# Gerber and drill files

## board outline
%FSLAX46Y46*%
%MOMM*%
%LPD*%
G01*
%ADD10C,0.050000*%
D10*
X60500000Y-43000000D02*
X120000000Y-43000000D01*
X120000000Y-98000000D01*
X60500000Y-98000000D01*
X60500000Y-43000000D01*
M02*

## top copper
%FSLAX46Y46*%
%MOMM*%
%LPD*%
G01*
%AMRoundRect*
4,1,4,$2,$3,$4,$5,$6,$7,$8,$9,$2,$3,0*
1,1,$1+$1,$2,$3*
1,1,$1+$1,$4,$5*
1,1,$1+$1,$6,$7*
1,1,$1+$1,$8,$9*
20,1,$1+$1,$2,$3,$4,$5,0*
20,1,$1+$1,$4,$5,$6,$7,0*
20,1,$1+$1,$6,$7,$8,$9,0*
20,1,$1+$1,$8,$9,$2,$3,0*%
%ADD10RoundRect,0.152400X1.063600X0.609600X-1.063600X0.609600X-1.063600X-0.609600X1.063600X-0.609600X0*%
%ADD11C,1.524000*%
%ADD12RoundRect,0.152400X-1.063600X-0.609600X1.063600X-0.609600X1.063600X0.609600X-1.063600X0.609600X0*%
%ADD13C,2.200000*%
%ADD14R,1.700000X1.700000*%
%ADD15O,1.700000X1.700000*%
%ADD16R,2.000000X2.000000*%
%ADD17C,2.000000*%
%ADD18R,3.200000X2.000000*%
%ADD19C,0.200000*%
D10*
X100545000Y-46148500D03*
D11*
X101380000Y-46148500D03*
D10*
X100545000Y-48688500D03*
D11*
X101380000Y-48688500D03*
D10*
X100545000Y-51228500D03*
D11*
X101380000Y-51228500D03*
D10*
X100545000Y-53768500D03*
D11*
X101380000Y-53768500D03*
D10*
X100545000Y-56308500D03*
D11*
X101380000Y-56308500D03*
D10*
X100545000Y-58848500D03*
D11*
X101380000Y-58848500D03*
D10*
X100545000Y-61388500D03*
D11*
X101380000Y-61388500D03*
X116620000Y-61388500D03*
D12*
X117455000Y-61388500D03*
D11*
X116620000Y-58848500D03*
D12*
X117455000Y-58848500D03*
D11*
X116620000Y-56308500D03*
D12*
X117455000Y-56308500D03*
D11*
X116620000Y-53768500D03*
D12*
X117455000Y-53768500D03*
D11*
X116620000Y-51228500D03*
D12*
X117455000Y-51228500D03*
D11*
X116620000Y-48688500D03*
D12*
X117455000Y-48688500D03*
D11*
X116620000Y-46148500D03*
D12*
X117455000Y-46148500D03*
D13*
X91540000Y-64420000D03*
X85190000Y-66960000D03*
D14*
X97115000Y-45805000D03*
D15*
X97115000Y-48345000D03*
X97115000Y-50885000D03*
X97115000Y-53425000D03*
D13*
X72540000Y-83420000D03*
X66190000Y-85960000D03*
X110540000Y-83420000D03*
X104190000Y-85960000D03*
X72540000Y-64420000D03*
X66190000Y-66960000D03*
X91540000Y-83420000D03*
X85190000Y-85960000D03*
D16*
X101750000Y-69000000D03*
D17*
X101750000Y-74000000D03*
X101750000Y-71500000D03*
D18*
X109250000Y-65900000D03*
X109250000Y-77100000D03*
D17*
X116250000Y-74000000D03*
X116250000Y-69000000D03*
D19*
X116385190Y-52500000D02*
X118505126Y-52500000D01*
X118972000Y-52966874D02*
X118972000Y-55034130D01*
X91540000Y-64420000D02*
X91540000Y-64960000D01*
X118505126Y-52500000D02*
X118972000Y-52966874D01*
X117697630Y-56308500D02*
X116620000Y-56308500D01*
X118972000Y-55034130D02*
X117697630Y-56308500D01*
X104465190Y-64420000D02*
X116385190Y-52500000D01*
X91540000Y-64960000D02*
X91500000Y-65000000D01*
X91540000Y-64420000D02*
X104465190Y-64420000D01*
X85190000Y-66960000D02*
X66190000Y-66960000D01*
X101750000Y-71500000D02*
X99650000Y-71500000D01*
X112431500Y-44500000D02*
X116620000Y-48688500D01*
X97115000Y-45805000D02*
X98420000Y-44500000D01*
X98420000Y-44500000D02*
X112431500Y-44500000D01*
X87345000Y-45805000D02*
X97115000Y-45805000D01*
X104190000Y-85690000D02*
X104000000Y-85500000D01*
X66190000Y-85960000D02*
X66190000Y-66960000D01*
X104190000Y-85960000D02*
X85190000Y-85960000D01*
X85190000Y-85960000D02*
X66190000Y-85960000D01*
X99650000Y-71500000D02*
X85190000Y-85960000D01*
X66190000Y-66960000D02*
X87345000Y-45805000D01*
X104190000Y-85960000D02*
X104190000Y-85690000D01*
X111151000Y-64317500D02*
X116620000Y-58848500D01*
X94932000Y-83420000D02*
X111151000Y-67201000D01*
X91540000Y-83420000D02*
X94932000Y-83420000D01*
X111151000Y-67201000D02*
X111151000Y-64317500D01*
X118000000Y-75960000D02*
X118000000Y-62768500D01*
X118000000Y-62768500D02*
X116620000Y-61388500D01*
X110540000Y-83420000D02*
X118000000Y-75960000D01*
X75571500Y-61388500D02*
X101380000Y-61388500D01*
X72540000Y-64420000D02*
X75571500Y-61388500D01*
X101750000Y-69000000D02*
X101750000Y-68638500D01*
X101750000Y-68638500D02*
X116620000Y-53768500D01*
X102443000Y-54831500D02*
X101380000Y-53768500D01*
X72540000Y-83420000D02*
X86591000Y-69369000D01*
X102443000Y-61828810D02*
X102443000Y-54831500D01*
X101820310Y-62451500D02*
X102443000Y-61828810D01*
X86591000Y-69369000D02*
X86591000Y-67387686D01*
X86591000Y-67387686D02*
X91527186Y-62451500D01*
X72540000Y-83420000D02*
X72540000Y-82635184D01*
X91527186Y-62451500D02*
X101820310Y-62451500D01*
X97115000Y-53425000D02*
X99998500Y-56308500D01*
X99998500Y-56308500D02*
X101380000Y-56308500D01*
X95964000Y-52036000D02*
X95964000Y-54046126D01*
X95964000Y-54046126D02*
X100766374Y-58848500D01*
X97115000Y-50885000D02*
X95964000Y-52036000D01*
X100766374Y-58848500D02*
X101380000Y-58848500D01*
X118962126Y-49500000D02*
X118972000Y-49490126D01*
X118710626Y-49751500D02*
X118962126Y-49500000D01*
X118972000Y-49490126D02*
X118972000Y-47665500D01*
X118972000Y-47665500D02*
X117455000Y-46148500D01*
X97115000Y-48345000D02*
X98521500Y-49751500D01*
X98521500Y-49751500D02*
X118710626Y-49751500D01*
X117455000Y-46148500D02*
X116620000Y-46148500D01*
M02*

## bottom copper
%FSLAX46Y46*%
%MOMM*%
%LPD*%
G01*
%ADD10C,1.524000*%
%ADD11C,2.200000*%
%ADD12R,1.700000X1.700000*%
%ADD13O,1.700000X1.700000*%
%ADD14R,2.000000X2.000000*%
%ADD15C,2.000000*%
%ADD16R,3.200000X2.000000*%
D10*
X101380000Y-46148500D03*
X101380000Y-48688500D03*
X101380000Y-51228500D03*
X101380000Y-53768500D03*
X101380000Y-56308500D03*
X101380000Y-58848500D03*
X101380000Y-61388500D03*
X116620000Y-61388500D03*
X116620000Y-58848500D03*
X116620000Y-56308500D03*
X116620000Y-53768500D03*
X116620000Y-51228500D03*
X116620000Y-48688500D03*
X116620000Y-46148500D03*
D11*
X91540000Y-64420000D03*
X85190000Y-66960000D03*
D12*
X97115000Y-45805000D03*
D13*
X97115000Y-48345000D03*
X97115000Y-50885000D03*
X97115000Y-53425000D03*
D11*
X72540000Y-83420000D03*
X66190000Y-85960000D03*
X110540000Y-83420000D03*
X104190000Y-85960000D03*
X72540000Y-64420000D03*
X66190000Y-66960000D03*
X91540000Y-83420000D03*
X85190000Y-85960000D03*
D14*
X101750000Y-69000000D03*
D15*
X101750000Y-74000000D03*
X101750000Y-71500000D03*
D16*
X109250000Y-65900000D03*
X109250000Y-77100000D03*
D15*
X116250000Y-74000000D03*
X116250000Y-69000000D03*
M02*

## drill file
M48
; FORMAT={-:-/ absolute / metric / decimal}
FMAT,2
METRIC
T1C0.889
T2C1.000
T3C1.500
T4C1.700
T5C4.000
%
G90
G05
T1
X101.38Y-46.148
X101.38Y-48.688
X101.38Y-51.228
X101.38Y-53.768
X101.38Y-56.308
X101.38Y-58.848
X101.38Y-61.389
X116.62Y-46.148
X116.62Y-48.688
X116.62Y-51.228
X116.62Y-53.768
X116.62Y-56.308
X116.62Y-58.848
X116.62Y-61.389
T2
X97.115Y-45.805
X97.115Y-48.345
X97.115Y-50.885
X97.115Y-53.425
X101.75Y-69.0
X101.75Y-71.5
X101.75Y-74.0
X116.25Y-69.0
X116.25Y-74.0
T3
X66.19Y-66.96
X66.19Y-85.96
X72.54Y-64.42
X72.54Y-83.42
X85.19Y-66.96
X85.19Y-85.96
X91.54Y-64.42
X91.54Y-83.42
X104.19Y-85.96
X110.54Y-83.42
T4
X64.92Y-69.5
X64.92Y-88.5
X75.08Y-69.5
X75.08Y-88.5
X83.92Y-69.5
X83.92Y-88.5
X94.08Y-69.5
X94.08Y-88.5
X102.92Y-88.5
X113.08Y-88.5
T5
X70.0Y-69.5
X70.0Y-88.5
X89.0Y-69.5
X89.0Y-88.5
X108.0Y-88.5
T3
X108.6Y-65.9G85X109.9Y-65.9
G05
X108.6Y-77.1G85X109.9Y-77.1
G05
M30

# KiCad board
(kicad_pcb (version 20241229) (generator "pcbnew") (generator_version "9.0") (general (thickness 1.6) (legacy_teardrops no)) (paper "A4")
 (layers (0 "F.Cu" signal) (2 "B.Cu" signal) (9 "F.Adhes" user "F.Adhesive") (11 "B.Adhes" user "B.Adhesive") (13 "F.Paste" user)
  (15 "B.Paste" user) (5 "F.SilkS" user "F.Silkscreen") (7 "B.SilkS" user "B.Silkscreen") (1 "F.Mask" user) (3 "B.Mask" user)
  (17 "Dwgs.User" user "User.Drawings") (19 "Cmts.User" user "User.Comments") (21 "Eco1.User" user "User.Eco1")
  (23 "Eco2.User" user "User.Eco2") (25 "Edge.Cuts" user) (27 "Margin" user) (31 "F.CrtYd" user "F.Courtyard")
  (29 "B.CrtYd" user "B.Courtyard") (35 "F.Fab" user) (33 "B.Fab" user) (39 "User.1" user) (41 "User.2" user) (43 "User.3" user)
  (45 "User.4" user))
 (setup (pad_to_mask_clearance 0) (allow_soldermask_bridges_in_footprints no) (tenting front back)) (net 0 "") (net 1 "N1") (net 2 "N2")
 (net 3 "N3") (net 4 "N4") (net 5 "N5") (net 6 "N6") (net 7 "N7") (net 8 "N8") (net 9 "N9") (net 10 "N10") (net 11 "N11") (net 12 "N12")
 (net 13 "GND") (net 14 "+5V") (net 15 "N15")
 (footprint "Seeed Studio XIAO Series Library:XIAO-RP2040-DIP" (layer "F.Cu") (at 109 53.7685)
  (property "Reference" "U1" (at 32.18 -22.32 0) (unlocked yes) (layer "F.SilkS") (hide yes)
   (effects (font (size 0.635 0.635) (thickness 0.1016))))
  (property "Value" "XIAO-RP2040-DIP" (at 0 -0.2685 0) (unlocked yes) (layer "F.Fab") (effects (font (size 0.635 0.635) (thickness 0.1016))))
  (pad "1" smd roundrect (at -8.455 -7.62 180) (size 2.432 1.524) (layers "F.Cu" "F.Mask") (roundrect_rratio 0.1) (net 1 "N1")
   (thermal_bridge_angle 45))
  (pad "1" thru_hole circle (at -7.62 -7.62 180) (size 1.524 1.524) (drill 0.889) (layers "*.Cu" "*.Mask") (remove_unused_layers no)
   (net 1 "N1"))
  (pad "2" smd roundrect (at -8.455 -5.08 180) (size 2.432 1.524) (layers "F.Cu" "F.Mask") (roundrect_rratio 0.1) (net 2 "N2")
   (thermal_bridge_angle 45))
  (pad "2" thru_hole circle (at -7.62 -5.08 180) (size 1.524 1.524) (drill 0.889) (layers "*.Cu" "*.Mask") (remove_unused_layers no)
   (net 2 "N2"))
  (pad "3" smd roundrect (at -8.455 -2.54 180) (size 2.432 1.524) (layers "F.Cu" "F.Mask") (roundrect_rratio 0.1) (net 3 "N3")
   (thermal_bridge_angle 45))
  (pad "3" thru_hole circle (at -7.62 -2.54 180) (size 1.524 1.524) (drill 0.889) (layers "*.Cu" "*.Mask") (remove_unused_layers no)
   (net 3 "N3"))
  (pad "4" smd roundrect (at -8.455 0 180) (size 2.432 1.524) (layers "F.Cu" "F.Mask") (roundrect_rratio 0.1) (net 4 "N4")
   (thermal_bridge_angle 45))
  (pad "4" thru_hole circle (at -7.62 0 180) (size 1.524 1.524) (drill 0.889) (layers "*.Cu" "*.Mask") (remove_unused_layers no)
   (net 4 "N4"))
  (pad "5" smd roundrect (at -8.455 2.54 180) (size 2.432 1.524) (layers "F.Cu" "F.Mask") (roundrect_rratio 0.1) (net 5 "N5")
   (thermal_bridge_angle 45))
  (pad "5" thru_hole circle (at -7.62 2.54 180) (size 1.524 1.524) (drill 0.889) (layers "*.Cu" "*.Mask") (remove_unused_layers no)
   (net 5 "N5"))
  (pad "6" smd roundrect (at -8.455 5.08 180) (size 2.432 1.524) (layers "F.Cu" "F.Mask") (roundrect_rratio 0.1) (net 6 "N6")
   (thermal_bridge_angle 45))
  (pad "6" thru_hole circle (at -7.62 5.08 180) (size 1.524 1.524) (drill 0.889) (layers "*.Cu" "*.Mask") (remove_unused_layers no)
   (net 6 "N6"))
  (pad "7" smd roundrect (at -8.455 7.62 180) (size 2.432 1.524) (layers "F.Cu" "F.Mask") (roundrect_rratio 0.1) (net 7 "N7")
   (thermal_bridge_angle 45))
  (pad "7" thru_hole circle (at -7.62 7.62 180) (size 1.524 1.524) (drill 0.889) (layers "*.Cu" "*.Mask") (remove_unused_layers no)
   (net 7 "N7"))
  (pad "8" thru_hole circle (at 7.62 7.62) (size 1.524 1.524) (drill 0.889) (layers "*.Cu" "*.Mask") (remove_unused_layers no) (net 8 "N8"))
  (pad "8" smd roundrect (at 8.455 7.62) (size 2.432 1.524) (layers "F.Cu" "F.Mask") (roundrect_rratio 0.1) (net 8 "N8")
   (thermal_bridge_angle 45))
  (pad "9" thru_hole circle (at 7.62 5.08) (size 1.524 1.524) (drill 0.889) (layers "*.Cu" "*.Mask") (remove_unused_layers no) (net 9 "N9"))
  (pad "9" smd roundrect (at 8.455 5.08) (size 2.432 1.524) (layers "F.Cu" "F.Mask") (roundrect_rratio 0.1) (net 9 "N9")
   (thermal_bridge_angle 45))
  (pad "10" thru_hole circle (at 7.62 2.54) (size 1.524 1.524) (drill 0.889) (layers "*.Cu" "*.Mask") (remove_unused_layers no)
   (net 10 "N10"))
  (pad "10" smd roundrect (at 8.455 2.54) (size 2.432 1.524) (layers "F.Cu" "F.Mask") (roundrect_rratio 0.1) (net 10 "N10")
   (thermal_bridge_angle 45))
  (pad "11" thru_hole circle (at 7.62 0) (size 1.524 1.524) (drill 0.889) (layers "*.Cu" "*.Mask") (remove_unused_layers no) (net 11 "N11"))
  (pad "11" smd roundrect (at 8.455 0) (size 2.432 1.524) (layers "F.Cu" "F.Mask") (roundrect_rratio 0.1) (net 11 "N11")
   (thermal_bridge_angle 45))
  (pad "12" thru_hole circle (at 7.62 -2.54) (size 1.524 1.524) (drill 0.889) (layers "*.Cu" "*.Mask") (remove_unused_layers no)
   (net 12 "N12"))
  (pad "12" smd roundrect (at 8.455 -2.54) (size 2.432 1.524) (layers "F.Cu" "F.Mask") (roundrect_rratio 0.1) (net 12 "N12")
   (thermal_bridge_angle 45))
  (pad "13" thru_hole circle (at 7.62 -5.08) (size 1.524 1.524) (drill 0.889) (layers "*.Cu" "*.Mask") (remove_unused_layers no)
   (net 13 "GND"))
  (pad "13" smd roundrect (at 8.455 -5.08) (size 2.432 1.524) (layers "F.Cu" "F.Mask") (roundrect_rratio 0.1) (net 13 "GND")
   (thermal_bridge_angle 45))
  (pad "14" thru_hole circle (at 7.62 -7.62) (size 1.524 1.524) (drill 0.889) (layers "*.Cu" "*.Mask") (remove_unused_layers no)
   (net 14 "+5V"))
  (pad "14" smd roundrect (at 8.455 -7.62) (size 2.432 1.524) (layers "F.Cu" "F.Mask") (roundrect_rratio 0.1) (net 14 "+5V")
   (thermal_bridge_angle 45)))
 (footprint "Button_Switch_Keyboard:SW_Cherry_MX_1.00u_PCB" (layer "F.Cu") (at 91.54 64.42)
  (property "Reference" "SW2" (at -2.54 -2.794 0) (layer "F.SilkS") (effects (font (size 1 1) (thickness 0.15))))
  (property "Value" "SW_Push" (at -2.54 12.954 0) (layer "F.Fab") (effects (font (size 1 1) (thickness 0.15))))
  (pad "" np_thru_hole circle (at -7.62 5.08) (size 1.7 1.7) (drill 1.7) (layers "*.Cu" "*.Mask"))
  (pad "" np_thru_hole circle (at -2.54 5.08) (size 4 4) (drill 4) (layers "*.Cu" "*.Mask"))
  (pad "" np_thru_hole circle (at 2.54 5.08) (size 1.7 1.7) (drill 1.7) (layers "*.Cu" "*.Mask"))
  (pad "1" thru_hole circle (at 0 0) (size 2.2 2.2) (drill 1.5) (layers "*.Cu" "*.Mask") (remove_unused_layers no) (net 10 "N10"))
  (pad "2" thru_hole circle (at -6.35 2.54) (size 2.2 2.2) (drill 1.5) (layers "*.Cu" "*.Mask") (remove_unused_layers no) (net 13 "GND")))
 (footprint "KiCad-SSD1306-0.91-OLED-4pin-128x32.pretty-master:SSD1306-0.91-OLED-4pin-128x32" (layer "F.Cu") (at 60.615 43.615)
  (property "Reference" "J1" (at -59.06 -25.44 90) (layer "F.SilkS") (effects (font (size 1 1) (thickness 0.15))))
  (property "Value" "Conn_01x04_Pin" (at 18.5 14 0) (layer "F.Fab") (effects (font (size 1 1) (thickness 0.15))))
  (pad "1" thru_hole rect (at 36.5 2.19) (size 1.7 1.7) (drill 1) (layers "*.Cu" "*.Mask") (remove_unused_layers no) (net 13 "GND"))
  (pad "2" thru_hole oval (at 36.5 4.73) (size 1.7 1.7) (drill 1) (layers "*.Cu" "*.Mask") (remove_unused_layers no) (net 14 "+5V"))
  (pad "3" thru_hole oval (at 36.5 7.27) (size 1.7 1.7) (drill 1) (layers "*.Cu" "*.Mask") (remove_unused_layers no) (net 6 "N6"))
  (pad "4" thru_hole oval (at 36.5 9.81) (size 1.7 1.7) (drill 1) (layers "*.Cu" "*.Mask") (remove_unused_layers no) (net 5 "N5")))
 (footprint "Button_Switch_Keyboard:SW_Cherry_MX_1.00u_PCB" (layer "F.Cu") (at 72.54 83.42)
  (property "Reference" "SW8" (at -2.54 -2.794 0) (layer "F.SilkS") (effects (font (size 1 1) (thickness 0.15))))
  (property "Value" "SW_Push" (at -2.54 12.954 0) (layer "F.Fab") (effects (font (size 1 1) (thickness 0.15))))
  (pad "" np_thru_hole circle (at -7.62 5.08) (size 1.7 1.7) (drill 1.7) (layers "*.Cu" "*.Mask"))
  (pad "" np_thru_hole circle (at -2.54 5.08) (size 4 4) (drill 4) (layers "*.Cu" "*.Mask"))
  (pad "" np_thru_hole circle (at 2.54 5.08) (size 1.7 1.7) (drill 1.7) (layers "*.Cu" "*.Mask"))
  (pad "1" thru_hole circle (at 0 0) (size 2.2 2.2) (drill 1.5) (layers "*.Cu" "*.Mask") (remove_unused_layers no) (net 4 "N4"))
  (pad "2" thru_hole circle (at -6.35 2.54) (size 2.2 2.2) (drill 1.5) (layers "*.Cu" "*.Mask") (remove_unused_layers no) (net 13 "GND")))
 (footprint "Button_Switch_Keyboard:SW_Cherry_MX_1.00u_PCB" (layer "F.Cu") (at 110.54 83.42)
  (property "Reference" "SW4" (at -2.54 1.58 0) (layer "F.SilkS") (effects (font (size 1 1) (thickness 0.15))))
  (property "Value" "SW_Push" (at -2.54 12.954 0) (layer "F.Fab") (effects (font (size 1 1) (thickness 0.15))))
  (pad "" np_thru_hole circle (at -7.62 5.08) (size 1.7 1.7) (drill 1.7) (layers "*.Cu" "*.Mask"))
  (pad "" np_thru_hole circle (at -2.54 5.08) (size 4 4) (drill 4) (layers "*.Cu" "*.Mask"))
  (pad "" np_thru_hole circle (at 2.54 5.08) (size 1.7 1.7) (drill 1.7) (layers "*.Cu" "*.Mask"))
  (pad "1" thru_hole circle (at 0 0) (size 2.2 2.2) (drill 1.5) (layers "*.Cu" "*.Mask") (remove_unused_layers no) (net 8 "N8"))
  (pad "2" thru_hole circle (at -6.35 2.54) (size 2.2 2.2) (drill 1.5) (layers "*.Cu" "*.Mask") (remove_unused_layers no) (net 13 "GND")))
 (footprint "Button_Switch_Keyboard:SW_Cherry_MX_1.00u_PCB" (layer "F.Cu") (at 72.54 64.42)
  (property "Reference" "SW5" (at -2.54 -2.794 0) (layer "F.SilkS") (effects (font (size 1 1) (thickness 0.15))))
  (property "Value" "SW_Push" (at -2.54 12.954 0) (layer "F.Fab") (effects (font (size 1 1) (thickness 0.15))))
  (pad "" np_thru_hole circle (at -7.62 5.08) (size 1.7 1.7) (drill 1.7) (layers "*.Cu" "*.Mask"))
  (pad "" np_thru_hole circle (at -2.54 5.08) (size 4 4) (drill 4) (layers "*.Cu" "*.Mask"))
  (pad "" np_thru_hole circle (at 2.54 5.08) (size 1.7 1.7) (drill 1.7) (layers "*.Cu" "*.Mask"))
  (pad "1" thru_hole circle (at 0 0) (size 2.2 2.2) (drill 1.5) (layers "*.Cu" "*.Mask") (remove_unused_layers no) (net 7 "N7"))
  (pad "2" thru_hole circle (at -6.35 2.54) (size 2.2 2.2) (drill 1.5) (layers "*.Cu" "*.Mask") (remove_unused_layers no) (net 13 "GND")))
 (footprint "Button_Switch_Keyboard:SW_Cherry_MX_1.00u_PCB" (layer "F.Cu") (at 91.54 83.42)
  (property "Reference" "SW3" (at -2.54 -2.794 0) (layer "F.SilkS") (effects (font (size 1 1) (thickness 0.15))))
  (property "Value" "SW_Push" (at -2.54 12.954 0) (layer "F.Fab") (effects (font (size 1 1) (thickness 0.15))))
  (pad "" np_thru_hole circle (at -7.62 5.08) (size 1.7 1.7) (drill 1.7) (layers "*.Cu" "*.Mask"))
  (pad "" np_thru_hole circle (at -2.54 5.08) (size 4 4) (drill 4) (layers "*.Cu" "*.Mask"))
  (pad "" np_thru_hole circle (at 2.54 5.08) (size 1.7 1.7) (drill 1.7) (layers "*.Cu" "*.Mask"))
  (pad "1" thru_hole circle (at 0 0) (size 2.2 2.2) (drill 1.5) (layers "*.Cu" "*.Mask") (remove_unused_layers no) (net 9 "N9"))
  (pad "2" thru_hole circle (at -6.35 2.54) (size 2.2 2.2) (drill 1.5) (layers "*.Cu" "*.Mask") (remove_unused_layers no) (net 13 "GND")))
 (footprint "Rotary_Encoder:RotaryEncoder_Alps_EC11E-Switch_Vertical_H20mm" (layer "F.Cu") (at 101.75 69)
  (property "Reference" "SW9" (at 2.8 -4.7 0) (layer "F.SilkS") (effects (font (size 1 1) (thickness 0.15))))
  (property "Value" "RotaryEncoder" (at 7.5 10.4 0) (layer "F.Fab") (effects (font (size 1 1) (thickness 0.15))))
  (pad "A" thru_hole rect (at 0 0) (size 2 2) (drill 1) (layers "*.Cu" "*.Mask") (remove_unused_layers no) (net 11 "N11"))
  (pad "B" thru_hole circle (at 0 5) (size 2 2) (drill 1) (layers "*.Cu" "*.Mask") (remove_unused_layers no) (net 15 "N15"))
  (pad "C" thru_hole circle (at 0 2.5) (size 2 2) (drill 1) (layers "*.Cu" "*.Mask") (remove_unused_layers no) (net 13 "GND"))
  (pad "MP" thru_hole rect (at 7.5 -3.1) (size 3.2 2) (drill oval 2.8 1.5) (layers "*.Cu" "*.Mask") (remove_unused_layers no))
  (pad "MP" thru_hole rect (at 7.5 8.1) (size 3.2 2) (drill oval 2.8 1.5) (layers "*.Cu" "*.Mask") (remove_unused_layers no))
  (pad "S1" thru_hole circle (at 14.5 5) (size 2 2) (drill 1) (layers "*.Cu" "*.Mask") (remove_unused_layers no))
  (pad "S2" thru_hole circle (at 14.5 0) (size 2 2) (drill 1) (layers "*.Cu" "*.Mask") (remove_unused_layers no)))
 (gr_rect (start 60.5 43) (end 120 98) (stroke (width 0.05) (type default)) (fill no) (layer "Edge.Cuts"))
 (segment (start 116.38519 52.5) (end 118.505126 52.5) (width 0.2) (layer "F.Cu") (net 10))
 (segment (start 118.972 52.966874) (end 118.972 55.03413) (width 0.2) (layer "F.Cu") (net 10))
 (segment (start 91.54 64.42) (end 91.54 64.96) (width 0.2) (layer "F.Cu") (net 10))
 (segment (start 118.505126 52.5) (end 118.972 52.966874) (width 0.2) (layer "F.Cu") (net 10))
 (segment (start 117.69763 56.3085) (end 116.62 56.3085) (width 0.2) (layer "F.Cu") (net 10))
 (segment (start 118.972 55.03413) (end 117.69763 56.3085) (width 0.2) (layer "F.Cu") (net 10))
 (segment (start 104.46519 64.42) (end 116.38519 52.5) (width 0.2) (layer "F.Cu") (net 10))
 (segment (start 91.54 64.96) (end 91.5 65) (width 0.2) (layer "F.Cu") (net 10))
 (segment (start 91.54 64.42) (end 104.46519 64.42) (width 0.2) (layer "F.Cu") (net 10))
 (segment (start 85.19 66.96) (end 66.19 66.96) (width 0.2) (layer "F.Cu") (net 13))
 (segment (start 101.75 71.5) (end 99.65 71.5) (width 0.2) (layer "F.Cu") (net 13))
 (segment (start 112.4315 44.5) (end 116.62 48.6885) (width 0.2) (layer "F.Cu") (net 13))
 (segment (start 97.115 45.805) (end 98.42 44.5) (width 0.2) (layer "F.Cu") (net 13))
 (segment (start 98.42 44.5) (end 112.4315 44.5) (width 0.2) (layer "F.Cu") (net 13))
 (segment (start 87.345 45.805) (end 97.115 45.805) (width 0.2) (layer "F.Cu") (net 13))
 (segment (start 104.19 85.69) (end 104 85.5) (width 0.2) (layer "F.Cu") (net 13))
 (segment (start 66.19 85.96) (end 66.19 66.96) (width 0.2) (layer "F.Cu") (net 13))
 (segment (start 104.19 85.96) (end 85.19 85.96) (width 0.2) (layer "F.Cu") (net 13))
 (segment (start 85.19 85.96) (end 66.19 85.96) (width 0.2) (layer "F.Cu") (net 13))
 (segment (start 99.65 71.5) (end 85.19 85.96) (width 0.2) (layer "F.Cu") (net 13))
 (segment (start 66.19 66.96) (end 87.345 45.805) (width 0.2) (layer "F.Cu") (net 13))
 (segment (start 104.19 85.96) (end 104.19 85.69) (width 0.2) (layer "F.Cu") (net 13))
 (segment (start 111.151 64.3175) (end 116.62 58.8485) (width 0.2) (layer "F.Cu") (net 9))
 (segment (start 94.932 83.42) (end 111.151 67.201) (width 0.2) (layer "F.Cu") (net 9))
 (segment (start 91.54 83.42) (end 94.932 83.42) (width 0.2) (layer "F.Cu") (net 9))
 (segment (start 111.151 67.201) (end 111.151 64.3175) (width 0.2) (layer "F.Cu") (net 9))
 (segment (start 118 75.96) (end 118 62.7685) (width 0.2) (layer "F.Cu") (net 8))
 (segment (start 118 62.7685) (end 116.62 61.3885) (width 0.2) (layer "F.Cu") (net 8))
 (segment (start 110.54 83.42) (end 118 75.96) (width 0.2) (layer "F.Cu") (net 8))
 (segment (start 75.5715 61.3885) (end 101.38 61.3885) (width 0.2) (layer "F.Cu") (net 7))
 (segment (start 72.54 64.42) (end 75.5715 61.3885) (width 0.2) (layer "F.Cu") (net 7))
 (segment (start 101.75 69) (end 101.75 68.6385) (width 0.2) (layer "F.Cu") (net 11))
 (segment (start 101.75 68.6385) (end 116.62 53.7685) (width 0.2) (layer "F.Cu") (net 11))
 (segment (start 102.443 54.8315) (end 101.38 53.7685) (width 0.2) (layer "F.Cu") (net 4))
 (segment (start 72.54 83.42) (end 86.591 69.369) (width 0.2) (layer "F.Cu") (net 4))
 (segment (start 102.443 61.82881) (end 102.443 54.8315) (width 0.2) (layer "F.Cu") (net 4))
 (segment (start 101.82031 62.4515) (end 102.443 61.82881) (width 0.2) (layer "F.Cu") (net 4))
 (segment (start 86.591 69.369) (end 86.591 67.387686) (width 0.2) (layer "F.Cu") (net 4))
 (segment (start 86.591 67.387686) (end 91.527186 62.4515) (width 0.2) (layer "F.Cu") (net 4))
 (segment (start 72.54 83.42) (end 72.54 82.635184) (width 0.2) (layer "F.Cu") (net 4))
 (segment (start 91.527186 62.4515) (end 101.82031 62.4515) (width 0.2) (layer "F.Cu") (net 4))
 (segment (start 97.115 53.425) (end 99.9985 56.3085) (width 0.2) (layer "F.Cu") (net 5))
 (segment (start 99.9985 56.3085) (end 101.38 56.3085) (width 0.2) (layer "F.Cu") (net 5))
 (segment (start 95.964 52.036) (end 95.964 54.046126) (width 0.2) (layer "F.Cu") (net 6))
 (segment (start 95.964 54.046126) (end 100.766374 58.8485) (width 0.2) (layer "F.Cu") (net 6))
 (segment (start 97.115 50.885) (end 95.964 52.036) (width 0.2) (layer "F.Cu") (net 6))
 (segment (start 100.766374 58.8485) (end 101.38 58.8485) (width 0.2) (layer "F.Cu") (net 6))
 (segment (start 118.962126 49.5) (end 118.972 49.490126) (width 0.2) (layer "F.Cu") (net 14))
 (segment (start 118.710626 49.7515) (end 118.962126 49.5) (width 0.2) (layer "F.Cu") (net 14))
 (segment (start 118.972 49.490126) (end 118.972 47.6655) (width 0.2) (layer "F.Cu") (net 14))
 (segment (start 118.972 47.6655) (end 117.455 46.1485) (width 0.2) (layer "F.Cu") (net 14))
 (segment (start 97.115 48.345) (end 98.5215 49.7515) (width 0.2) (layer "F.Cu") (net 14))
 (segment (start 98.5215 49.7515) (end 118.710626 49.7515) (width 0.2) (layer "F.Cu") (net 14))
 (segment (start 117.455 46.1485) (end 116.62 46.1485) (width 0.2) (layer "F.Cu") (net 14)))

